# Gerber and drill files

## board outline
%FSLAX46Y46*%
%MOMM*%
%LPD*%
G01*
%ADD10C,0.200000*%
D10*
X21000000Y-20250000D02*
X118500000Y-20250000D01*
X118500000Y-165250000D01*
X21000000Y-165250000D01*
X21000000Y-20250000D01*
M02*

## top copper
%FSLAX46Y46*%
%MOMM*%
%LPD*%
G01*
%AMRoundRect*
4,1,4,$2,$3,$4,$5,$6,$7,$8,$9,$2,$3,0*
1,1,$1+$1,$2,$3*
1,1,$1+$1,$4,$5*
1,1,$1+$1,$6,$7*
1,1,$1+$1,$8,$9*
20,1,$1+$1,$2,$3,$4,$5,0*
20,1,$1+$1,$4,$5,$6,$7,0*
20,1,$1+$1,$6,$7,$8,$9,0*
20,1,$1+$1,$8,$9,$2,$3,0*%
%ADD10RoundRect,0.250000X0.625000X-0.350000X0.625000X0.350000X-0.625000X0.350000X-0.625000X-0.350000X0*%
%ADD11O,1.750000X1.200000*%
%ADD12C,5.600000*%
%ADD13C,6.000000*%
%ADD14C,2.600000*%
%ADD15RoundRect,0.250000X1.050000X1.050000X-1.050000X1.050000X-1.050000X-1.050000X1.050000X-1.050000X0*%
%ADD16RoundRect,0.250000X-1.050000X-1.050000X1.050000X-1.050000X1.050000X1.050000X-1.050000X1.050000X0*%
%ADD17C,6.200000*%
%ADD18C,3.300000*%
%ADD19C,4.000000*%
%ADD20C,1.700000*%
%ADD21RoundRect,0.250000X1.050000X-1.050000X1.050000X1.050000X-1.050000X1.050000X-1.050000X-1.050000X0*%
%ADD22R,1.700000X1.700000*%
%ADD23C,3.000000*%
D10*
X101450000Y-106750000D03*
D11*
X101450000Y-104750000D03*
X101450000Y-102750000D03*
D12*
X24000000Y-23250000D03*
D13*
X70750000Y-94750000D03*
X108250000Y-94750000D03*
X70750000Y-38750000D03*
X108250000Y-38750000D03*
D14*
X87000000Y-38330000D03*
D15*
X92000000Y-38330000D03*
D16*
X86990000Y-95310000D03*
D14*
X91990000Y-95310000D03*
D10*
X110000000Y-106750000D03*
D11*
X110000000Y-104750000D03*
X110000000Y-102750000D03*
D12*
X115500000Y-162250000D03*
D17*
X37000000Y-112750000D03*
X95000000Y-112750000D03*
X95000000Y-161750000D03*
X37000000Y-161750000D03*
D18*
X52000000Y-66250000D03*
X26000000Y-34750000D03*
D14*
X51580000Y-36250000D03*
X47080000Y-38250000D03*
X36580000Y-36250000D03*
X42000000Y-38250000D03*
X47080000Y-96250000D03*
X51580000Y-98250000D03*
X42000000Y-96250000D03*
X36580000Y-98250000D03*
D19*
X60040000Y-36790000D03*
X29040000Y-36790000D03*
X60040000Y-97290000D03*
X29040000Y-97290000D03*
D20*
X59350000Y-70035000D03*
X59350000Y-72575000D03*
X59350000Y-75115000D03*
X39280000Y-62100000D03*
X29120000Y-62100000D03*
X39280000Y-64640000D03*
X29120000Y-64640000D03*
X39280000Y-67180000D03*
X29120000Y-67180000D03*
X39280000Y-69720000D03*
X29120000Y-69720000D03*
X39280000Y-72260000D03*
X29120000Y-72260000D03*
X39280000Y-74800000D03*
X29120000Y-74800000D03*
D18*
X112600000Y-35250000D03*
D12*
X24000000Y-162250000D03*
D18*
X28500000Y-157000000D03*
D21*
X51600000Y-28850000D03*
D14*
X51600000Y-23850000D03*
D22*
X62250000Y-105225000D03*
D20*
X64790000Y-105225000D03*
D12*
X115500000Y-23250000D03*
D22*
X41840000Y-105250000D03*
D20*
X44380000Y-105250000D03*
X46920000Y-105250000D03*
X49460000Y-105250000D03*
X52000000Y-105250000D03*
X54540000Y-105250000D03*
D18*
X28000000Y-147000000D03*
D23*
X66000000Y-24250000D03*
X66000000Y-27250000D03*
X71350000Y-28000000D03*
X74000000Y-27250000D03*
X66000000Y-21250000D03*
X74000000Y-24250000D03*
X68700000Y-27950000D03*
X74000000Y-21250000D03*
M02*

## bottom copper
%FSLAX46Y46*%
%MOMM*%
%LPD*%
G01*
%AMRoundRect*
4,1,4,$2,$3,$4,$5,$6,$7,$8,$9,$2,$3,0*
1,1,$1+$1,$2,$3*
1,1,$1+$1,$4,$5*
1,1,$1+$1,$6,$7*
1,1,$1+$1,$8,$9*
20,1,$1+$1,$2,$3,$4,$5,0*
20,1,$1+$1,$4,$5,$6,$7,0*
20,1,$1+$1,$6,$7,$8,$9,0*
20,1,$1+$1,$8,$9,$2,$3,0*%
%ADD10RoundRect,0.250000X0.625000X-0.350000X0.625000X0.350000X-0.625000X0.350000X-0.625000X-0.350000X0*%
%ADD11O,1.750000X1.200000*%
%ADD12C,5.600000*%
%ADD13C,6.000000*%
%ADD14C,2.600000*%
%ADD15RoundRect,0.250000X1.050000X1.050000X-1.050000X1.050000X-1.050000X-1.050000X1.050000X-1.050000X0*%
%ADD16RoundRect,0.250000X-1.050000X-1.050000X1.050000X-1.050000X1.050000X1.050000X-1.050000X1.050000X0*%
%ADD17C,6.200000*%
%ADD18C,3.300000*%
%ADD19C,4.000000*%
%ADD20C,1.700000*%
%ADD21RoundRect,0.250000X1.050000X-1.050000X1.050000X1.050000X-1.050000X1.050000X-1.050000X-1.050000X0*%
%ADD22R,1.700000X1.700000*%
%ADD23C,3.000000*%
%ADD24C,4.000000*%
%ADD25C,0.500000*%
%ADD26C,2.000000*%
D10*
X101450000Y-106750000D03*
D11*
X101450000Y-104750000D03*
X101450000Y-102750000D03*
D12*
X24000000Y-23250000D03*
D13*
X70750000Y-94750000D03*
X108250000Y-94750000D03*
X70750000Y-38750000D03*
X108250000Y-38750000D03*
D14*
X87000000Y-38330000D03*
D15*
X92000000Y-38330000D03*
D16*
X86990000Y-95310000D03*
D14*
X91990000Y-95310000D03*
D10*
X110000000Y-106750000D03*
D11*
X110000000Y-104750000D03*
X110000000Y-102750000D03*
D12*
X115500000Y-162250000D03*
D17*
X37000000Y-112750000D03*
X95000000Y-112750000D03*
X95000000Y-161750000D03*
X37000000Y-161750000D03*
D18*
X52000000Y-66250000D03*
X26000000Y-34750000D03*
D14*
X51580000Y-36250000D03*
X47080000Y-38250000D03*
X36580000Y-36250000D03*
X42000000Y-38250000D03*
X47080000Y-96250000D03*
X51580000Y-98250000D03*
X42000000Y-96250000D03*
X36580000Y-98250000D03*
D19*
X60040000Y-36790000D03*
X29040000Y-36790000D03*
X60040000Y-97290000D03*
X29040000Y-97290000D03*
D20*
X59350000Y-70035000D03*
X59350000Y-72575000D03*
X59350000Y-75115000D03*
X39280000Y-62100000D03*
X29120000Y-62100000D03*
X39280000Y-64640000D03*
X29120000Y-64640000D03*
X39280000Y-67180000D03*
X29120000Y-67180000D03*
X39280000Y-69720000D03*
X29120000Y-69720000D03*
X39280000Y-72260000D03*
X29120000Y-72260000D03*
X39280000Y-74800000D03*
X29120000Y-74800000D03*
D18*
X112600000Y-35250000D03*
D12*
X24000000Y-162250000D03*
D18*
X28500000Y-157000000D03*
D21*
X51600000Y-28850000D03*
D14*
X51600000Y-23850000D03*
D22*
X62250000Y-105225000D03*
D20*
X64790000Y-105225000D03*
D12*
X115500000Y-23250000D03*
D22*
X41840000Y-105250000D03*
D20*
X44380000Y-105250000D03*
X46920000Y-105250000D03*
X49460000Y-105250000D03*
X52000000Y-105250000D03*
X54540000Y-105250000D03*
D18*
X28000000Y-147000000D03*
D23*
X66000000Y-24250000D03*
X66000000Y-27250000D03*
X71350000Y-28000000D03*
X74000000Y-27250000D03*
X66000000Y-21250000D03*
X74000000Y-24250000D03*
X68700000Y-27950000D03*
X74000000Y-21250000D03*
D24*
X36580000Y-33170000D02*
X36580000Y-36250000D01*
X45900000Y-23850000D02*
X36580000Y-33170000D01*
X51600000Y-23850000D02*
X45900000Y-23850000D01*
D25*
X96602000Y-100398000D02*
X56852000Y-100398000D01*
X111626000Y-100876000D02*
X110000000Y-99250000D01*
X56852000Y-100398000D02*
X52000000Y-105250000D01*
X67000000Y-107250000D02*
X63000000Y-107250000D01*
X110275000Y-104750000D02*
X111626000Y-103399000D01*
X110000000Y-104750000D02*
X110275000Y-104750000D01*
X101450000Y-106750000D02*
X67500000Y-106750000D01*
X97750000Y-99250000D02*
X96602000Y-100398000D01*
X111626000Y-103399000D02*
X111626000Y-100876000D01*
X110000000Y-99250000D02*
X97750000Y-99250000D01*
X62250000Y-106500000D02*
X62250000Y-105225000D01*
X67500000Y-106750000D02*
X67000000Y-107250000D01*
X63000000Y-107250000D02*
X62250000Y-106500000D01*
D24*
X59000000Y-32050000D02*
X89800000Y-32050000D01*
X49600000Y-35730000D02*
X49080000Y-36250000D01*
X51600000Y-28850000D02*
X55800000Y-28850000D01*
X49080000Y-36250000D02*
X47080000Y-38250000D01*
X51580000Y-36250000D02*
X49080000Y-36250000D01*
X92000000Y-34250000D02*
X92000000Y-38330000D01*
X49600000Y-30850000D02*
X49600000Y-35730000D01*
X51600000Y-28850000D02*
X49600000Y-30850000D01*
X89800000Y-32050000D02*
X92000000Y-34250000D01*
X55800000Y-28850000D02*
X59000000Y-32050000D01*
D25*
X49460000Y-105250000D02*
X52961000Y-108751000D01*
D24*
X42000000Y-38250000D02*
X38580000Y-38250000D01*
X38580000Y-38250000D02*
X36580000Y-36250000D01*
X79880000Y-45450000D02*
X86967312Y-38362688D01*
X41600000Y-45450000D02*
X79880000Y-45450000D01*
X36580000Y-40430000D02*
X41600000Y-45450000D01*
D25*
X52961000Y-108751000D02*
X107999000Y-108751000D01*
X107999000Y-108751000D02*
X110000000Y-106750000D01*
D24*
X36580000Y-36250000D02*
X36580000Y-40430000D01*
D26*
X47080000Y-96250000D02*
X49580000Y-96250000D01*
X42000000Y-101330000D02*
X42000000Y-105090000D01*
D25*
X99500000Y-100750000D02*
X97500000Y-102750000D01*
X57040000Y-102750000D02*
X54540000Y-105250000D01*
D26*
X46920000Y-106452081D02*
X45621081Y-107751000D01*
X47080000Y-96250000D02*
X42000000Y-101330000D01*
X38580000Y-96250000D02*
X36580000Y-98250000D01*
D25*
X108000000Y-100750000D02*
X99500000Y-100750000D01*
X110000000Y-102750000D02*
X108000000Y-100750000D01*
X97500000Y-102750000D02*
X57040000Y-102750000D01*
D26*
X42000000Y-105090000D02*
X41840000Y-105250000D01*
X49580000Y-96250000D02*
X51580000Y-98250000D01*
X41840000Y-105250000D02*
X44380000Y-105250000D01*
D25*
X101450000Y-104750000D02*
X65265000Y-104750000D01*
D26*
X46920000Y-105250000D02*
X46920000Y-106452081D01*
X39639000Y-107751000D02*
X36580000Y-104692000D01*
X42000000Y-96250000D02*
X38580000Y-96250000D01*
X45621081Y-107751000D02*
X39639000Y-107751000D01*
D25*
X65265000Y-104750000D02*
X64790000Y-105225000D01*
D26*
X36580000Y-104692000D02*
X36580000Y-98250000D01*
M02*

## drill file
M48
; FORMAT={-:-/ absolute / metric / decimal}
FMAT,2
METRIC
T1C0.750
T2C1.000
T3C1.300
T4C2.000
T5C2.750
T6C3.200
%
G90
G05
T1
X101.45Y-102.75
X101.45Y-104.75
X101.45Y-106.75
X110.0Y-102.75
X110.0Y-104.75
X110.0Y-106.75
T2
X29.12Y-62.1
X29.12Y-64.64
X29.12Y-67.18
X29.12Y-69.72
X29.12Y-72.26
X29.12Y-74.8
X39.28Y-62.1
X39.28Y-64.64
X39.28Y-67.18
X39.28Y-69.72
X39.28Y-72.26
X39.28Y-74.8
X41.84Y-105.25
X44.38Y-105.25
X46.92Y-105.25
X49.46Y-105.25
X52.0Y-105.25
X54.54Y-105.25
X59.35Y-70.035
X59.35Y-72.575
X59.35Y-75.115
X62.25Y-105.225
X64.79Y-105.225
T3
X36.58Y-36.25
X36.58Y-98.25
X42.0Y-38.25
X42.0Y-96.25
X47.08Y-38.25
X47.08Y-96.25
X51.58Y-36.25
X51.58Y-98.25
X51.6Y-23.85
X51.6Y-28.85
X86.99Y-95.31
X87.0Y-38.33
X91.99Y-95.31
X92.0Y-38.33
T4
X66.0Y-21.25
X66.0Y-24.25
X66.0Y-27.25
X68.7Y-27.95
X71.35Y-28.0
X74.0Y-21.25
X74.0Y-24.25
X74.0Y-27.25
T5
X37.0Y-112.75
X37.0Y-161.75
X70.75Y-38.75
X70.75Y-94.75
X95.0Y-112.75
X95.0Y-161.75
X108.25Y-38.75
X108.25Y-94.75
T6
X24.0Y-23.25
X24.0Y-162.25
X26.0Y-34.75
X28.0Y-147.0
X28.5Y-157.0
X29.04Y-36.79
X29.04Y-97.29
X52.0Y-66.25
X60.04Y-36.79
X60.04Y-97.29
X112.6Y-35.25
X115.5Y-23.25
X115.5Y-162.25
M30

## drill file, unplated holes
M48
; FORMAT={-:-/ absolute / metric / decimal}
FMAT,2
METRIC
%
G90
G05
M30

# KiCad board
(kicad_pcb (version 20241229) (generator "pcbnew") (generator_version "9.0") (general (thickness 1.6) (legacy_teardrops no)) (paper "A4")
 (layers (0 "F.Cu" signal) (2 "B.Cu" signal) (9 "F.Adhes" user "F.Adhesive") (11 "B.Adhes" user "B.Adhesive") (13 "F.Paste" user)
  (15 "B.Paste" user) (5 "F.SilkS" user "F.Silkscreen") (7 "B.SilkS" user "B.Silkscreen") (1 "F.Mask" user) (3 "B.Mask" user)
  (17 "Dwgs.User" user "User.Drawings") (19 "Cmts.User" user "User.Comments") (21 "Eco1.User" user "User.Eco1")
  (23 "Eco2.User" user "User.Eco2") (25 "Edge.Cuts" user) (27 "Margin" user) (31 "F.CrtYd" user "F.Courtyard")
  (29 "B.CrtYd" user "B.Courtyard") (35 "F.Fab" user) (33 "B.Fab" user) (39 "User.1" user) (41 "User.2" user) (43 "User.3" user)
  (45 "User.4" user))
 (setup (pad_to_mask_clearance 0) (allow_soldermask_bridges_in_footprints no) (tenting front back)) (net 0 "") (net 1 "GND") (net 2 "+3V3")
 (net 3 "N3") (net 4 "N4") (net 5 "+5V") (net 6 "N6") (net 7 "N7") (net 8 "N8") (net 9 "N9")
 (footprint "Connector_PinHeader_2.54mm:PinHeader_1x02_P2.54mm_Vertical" (layer "F.Cu") (at 62.25 105.225 90)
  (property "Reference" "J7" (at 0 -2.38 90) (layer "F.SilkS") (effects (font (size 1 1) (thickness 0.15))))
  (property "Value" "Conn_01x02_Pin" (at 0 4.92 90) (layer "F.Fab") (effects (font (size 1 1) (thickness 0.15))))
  (pad "1" thru_hole rect (at 0 0 90) (size 1.7 1.7) (drill 1) (layers "*.Cu" "*.Mask") (remove_unused_layers no) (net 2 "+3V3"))
  (pad "2" thru_hole circle (at 0 2.54 90) (size 1.7 1.7) (drill 1) (layers "*.Cu" "*.Mask") (remove_unused_layers no) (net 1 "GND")))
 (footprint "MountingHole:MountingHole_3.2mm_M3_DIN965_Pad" (layer "F.Cu") (at 24 23.25)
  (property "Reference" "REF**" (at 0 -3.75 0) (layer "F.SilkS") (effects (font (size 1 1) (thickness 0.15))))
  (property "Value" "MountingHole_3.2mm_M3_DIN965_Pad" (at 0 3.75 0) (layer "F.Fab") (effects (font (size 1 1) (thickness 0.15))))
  (pad "1" thru_hole circle (at 0 0) (size 5.6 5.6) (drill 3.2) (layers "*.Cu" "*.Mask") (remove_unused_layers no) (zone_connect 2)))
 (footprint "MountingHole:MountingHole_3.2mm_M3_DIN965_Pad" (layer "F.Cu") (at 24 162.25)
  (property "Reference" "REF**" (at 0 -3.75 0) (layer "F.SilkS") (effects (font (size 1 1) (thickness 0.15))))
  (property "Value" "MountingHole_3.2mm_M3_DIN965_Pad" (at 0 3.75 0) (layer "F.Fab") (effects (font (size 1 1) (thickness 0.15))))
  (pad "1" thru_hole circle (at 0 0) (size 5.6 5.6) (drill 3.2) (layers "*.Cu" "*.Mask") (remove_unused_layers no) (zone_connect 2)))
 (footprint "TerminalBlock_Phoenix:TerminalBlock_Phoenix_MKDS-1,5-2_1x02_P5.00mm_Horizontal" (layer "F.Cu") (at 51.6 28.85 90)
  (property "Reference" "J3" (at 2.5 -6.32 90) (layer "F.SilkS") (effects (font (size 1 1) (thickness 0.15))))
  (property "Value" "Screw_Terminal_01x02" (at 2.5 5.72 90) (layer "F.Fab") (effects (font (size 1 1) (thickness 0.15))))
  (pad "1" thru_hole roundrect (at 0 0 90) (size 2.6 2.6) (drill 1.3) (layers "*.Cu" "*.Mask") (remove_unused_layers no)
   (roundrect_rratio 0.096154) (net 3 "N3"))
  (pad "2" thru_hole circle (at 5 0 90) (size 2.6 2.6) (drill 1.3) (layers "*.Cu" "*.Mask") (remove_unused_layers no) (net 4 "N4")))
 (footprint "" (layer "F.Cu") (at 28 147)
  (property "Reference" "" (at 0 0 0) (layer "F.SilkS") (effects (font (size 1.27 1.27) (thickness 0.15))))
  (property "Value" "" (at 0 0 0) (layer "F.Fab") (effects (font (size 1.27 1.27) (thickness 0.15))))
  (pad "1" thru_hole circle (at 0 0) (size 3.3 3.3) (drill 3.2) (layers "*.Cu" "*.Mask") (remove_unused_layers no) (zone_connect 2)))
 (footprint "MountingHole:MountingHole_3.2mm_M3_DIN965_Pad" (layer "F.Cu") (at 112.6 35.25)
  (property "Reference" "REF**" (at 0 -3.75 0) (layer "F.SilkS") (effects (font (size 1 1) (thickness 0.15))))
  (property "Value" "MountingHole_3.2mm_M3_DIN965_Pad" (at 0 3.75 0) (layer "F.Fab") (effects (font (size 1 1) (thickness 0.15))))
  (pad "1" thru_hole circle (at 0 0) (size 3.3 3.3) (drill 3.2) (layers "*.Cu" "*.Mask") (remove_unused_layers no) (zone_connect 2)))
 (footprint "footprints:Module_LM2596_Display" (layer "F.Cu") (at 62.58 67.25 -90)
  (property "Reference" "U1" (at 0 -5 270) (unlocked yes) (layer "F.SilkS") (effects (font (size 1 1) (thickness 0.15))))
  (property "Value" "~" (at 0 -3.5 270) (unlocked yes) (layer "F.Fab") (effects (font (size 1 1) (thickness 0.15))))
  (pad "1" thru_hole circle (at -31 11 270) (size 2.6 2.6) (drill 1.3) (layers "*.Cu" "*.Mask") (remove_unused_layers no) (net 3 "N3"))
  (pad "1" thru_hole circle (at -29 15.5 270) (size 2.6 2.6) (drill 1.3) (layers "*.Cu" "*.Mask") (remove_unused_layers no) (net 3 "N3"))
  (pad "2" thru_hole circle (at -31 26 270) (size 2.6 2.6) (drill 1.3) (layers "*.Cu" "*.Mask") (remove_unused_layers no) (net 4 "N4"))
  (pad "2" thru_hole circle (at -29 20.58 270) (size 2.6 2.6) (drill 1.3) (layers "*.Cu" "*.Mask") (remove_unused_layers no) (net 4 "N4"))
  (pad "3" thru_hole circle (at 29 15.5 270) (size 2.6 2.6) (drill 1.3) (layers "*.Cu" "*.Mask") (remove_unused_layers no) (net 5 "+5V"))
  (pad "3" thru_hole circle (at 31 11 270) (size 2.6 2.6) (drill 1.3) (layers "*.Cu" "*.Mask") (remove_unused_layers no) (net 5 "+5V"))
  (pad "4" thru_hole circle (at 29 20.58 270) (size 2.6 2.6) (drill 1.3) (layers "*.Cu" "*.Mask") (remove_unused_layers no) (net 1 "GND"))
  (pad "4" thru_hole circle (at 31 26 270) (size 2.6 2.6) (drill 1.3) (layers "*.Cu" "*.Mask") (remove_unused_layers no) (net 1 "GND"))
  (pad "5" thru_hole circle (at -30.46 2.54 270) (size 4 4) (drill 3.2) (layers "*.Cu" "*.Mask") (remove_unused_layers no))
  (pad "5" thru_hole circle (at -30.46 33.54 270) (size 4 4) (drill 3.2) (layers "*.Cu" "*.Mask") (remove_unused_layers no))
  (pad "5" thru_hole circle (at 30.04 2.54 270) (size 4 4) (drill 3.2) (layers "*.Cu" "*.Mask") (remove_unused_layers no))
  (pad "5" thru_hole circle (at 30.04 33.54 270) (size 4 4) (drill 3.2) (layers "*.Cu" "*.Mask") (remove_unused_layers no))
  (pad "6" thru_hole circle (at 2.785 3.23 90) (size 1.7 1.7) (drill 1) (layers "*.Cu" "*.Mask") (remove_unused_layers no))
  (pad "7" thru_hole circle (at 5.325 3.23 90) (size 1.7 1.7) (drill 1) (layers "*.Cu" "*.Mask") (remove_unused_layers no))
  (pad "8" thru_hole circle (at 7.865 3.23 90) (size 1.7 1.7) (drill 1) (layers "*.Cu" "*.Mask") (remove_unused_layers no))
  (pad "9" thru_hole circle (at -5.15 23.3 270) (size 1.7 1.7) (drill 1) (layers "*.Cu" "*.Mask") (remove_unused_layers no))
  (pad "9" thru_hole circle (at -5.15 33.46 270) (size 1.7 1.7) (drill 1) (layers "*.Cu" "*.Mask") (remove_unused_layers no))
  (pad "9" thru_hole circle (at -2.61 23.3 270) (size 1.7 1.7) (drill 1) (layers "*.Cu" "*.Mask") (remove_unused_layers no))
  (pad "9" thru_hole circle (at -2.61 33.46 270) (size 1.7 1.7) (drill 1) (layers "*.Cu" "*.Mask") (remove_unused_layers no))
  (pad "9" thru_hole circle (at -0.07 23.3 270) (size 1.7 1.7) (drill 1) (layers "*.Cu" "*.Mask") (remove_unused_layers no))
  (pad "9" thru_hole circle (at -0.07 33.46 270) (size 1.7 1.7) (drill 1) (layers "*.Cu" "*.Mask") (remove_unused_layers no))
  (pad "9" thru_hole circle (at 2.47 23.3 270) (size 1.7 1.7) (drill 1) (layers "*.Cu" "*.Mask" "Eco1.User") (remove_unused_layers no))
  (pad "9" thru_hole circle (at 2.47 33.46 270) (size 1.7 1.7) (drill 1) (layers "*.Cu" "*.Mask") (remove_unused_layers no))
  (pad "9" thru_hole circle (at 5.01 23.3 270) (size 1.7 1.7) (drill 1) (layers "*.Cu" "*.Mask") (remove_unused_layers no))
  (pad "9" thru_hole circle (at 5.01 33.46 270) (size 1.7 1.7) (drill 1) (layers "*.Cu" "*.Mask") (remove_unused_layers no))
  (pad "9" thru_hole circle (at 7.55 23.3 270) (size 1.7 1.7) (drill 1) (layers "*.Cu" "*.Mask") (remove_unused_layers no))
  (pad "9" thru_hole circle (at 7.55 33.46 270) (size 1.7 1.7) (drill 1) (layers "*.Cu" "*.Mask") (remove_unused_layers no)))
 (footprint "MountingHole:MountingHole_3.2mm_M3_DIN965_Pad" (layer "F.Cu") (at 115.5 162.25)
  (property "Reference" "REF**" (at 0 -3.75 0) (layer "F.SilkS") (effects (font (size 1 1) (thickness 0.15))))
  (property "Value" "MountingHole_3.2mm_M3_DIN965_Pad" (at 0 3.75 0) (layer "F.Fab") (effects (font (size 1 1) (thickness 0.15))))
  (pad "1" thru_hole circle (at 0 0) (size 5.6 5.6) (drill 3.2) (layers "*.Cu" "*.Mask") (remove_unused_layers no) (zone_connect 2)))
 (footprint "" (layer "F.Cu") (at 28.5 157)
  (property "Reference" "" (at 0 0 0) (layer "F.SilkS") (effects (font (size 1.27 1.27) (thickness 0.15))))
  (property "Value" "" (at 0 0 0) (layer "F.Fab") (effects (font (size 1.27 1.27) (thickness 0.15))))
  (pad "1" thru_hole circle (at 0 0) (size 3.3 3.3) (drill 3.2) (layers "*.Cu" "*.Mask") (remove_unused_layers no) (zone_connect 2)))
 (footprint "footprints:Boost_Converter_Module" (layer "F.Cu") (at 89.5 66.75 90)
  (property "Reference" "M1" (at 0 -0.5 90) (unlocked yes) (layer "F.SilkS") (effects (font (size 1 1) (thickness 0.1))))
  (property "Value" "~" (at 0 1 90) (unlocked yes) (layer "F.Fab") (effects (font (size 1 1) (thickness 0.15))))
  (pad "" thru_hole circle (at -28 -18.75 90) (size 6 6) (drill 2.75) (layers "*.Cu" "*.Mask") (remove_unused_layers no))
  (pad "" thru_hole circle (at -28 18.75 90) (size 6 6) (drill 2.75) (layers "*.Cu" "*.Mask") (remove_unused_layers no))
  (pad "" thru_hole circle (at 28 -18.75 90) (size 6 6) (drill 2.75) (layers "*.Cu" "*.Mask") (remove_unused_layers no))
  (pad "" thru_hole circle (at 28 18.75 90) (size 6 6) (drill 2.75) (layers "*.Cu" "*.Mask") (remove_unused_layers no))
  (pad "1" thru_hole circle (at 28.42 -2.5 180) (size 2.6 2.6) (drill 1.3) (layers "*.Cu" "*.Mask") (remove_unused_layers no) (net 4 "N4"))
  (pad "2" thru_hole roundrect (at 28.42 2.5 180) (size 2.6 2.6) (drill 1.3) (layers "*.Cu" "*.Mask") (remove_unused_layers no)
   (roundrect_rratio 0.096154) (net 3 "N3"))
  (pad "3" thru_hole roundrect (at -28.56 -2.51) (size 2.6 2.6) (drill 1.3) (layers "*.Cu" "*.Mask") (remove_unused_layers no)
   (roundrect_rratio 0.096154))
  (pad "4" thru_hole circle (at -28.56 2.49) (size 2.6 2.6) (drill 1.3) (layers "*.Cu" "*.Mask") (remove_unused_layers no)))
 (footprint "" (layer "F.Cu") (at 26 34.75)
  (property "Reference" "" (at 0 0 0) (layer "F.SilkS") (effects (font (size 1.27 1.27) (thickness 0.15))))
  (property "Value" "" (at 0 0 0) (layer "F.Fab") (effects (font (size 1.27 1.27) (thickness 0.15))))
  (pad "1" thru_hole circle (at 0 0) (size 3.3 3.3) (drill 3.2) (layers "*.Cu" "*.Mask") (remove_unused_layers no) (zone_connect 2)))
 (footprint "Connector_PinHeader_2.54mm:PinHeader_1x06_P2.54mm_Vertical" (layer "F.Cu") (at 41.84 105.25 90)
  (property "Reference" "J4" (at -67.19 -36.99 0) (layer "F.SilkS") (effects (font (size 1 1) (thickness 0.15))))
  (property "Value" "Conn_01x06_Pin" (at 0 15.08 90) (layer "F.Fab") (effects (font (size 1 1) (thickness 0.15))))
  (pad "1" thru_hole rect (at 0 0 90) (size 1.7 1.7) (drill 1) (layers "*.Cu" "*.Mask") (remove_unused_layers no) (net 5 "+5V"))
  (pad "2" thru_hole circle (at 0 2.54 90) (size 1.7 1.7) (drill 1) (layers "*.Cu" "*.Mask") (remove_unused_layers no) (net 5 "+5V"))
  (pad "3" thru_hole circle (at 0 5.08 90) (size 1.7 1.7) (drill 1) (layers "*.Cu" "*.Mask") (remove_unused_layers no) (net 1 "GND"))
  (pad "4" thru_hole circle (at 0 7.62 90) (size 1.7 1.7) (drill 1) (layers "*.Cu" "*.Mask") (remove_unused_layers no) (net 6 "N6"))
  (pad "5" thru_hole circle (at 0 10.16 90) (size 1.7 1.7) (drill 1) (layers "*.Cu" "*.Mask") (remove_unused_layers no) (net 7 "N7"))
  (pad "6" thru_hole circle (at 0 12.7 90) (size 1.7 1.7) (drill 1) (layers "*.Cu" "*.Mask") (remove_unused_layers no) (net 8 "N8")))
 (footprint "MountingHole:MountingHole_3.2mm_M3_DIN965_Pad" (layer "F.Cu") (at 115.5 23.25)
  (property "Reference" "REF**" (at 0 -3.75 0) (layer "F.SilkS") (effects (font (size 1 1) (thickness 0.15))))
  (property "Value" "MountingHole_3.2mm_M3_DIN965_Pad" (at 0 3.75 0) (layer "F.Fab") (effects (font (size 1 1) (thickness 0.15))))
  (pad "1" thru_hole circle (at 0 0) (size 5.6 5.6) (drill 3.2) (layers "*.Cu" "*.Mask") (remove_unused_layers no) (zone_connect 2)))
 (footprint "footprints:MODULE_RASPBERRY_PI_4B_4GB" (layer "F.Cu") (at 76 137.25)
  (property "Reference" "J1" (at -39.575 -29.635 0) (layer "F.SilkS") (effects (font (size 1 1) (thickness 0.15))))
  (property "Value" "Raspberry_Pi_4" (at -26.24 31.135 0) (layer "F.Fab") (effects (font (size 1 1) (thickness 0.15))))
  (pad "S1" thru_hole circle (at -39 -24.5) (size 6.2 6.2) (drill 2.75) (layers "*.Cu" "*.Mask") (remove_unused_layers no)
   (solder_mask_margin 0.102))
  (pad "S2" thru_hole circle (at 19 -24.5) (size 6.2 6.2) (drill 2.75) (layers "*.Cu" "*.Mask") (remove_unused_layers no)
   (solder_mask_margin 0.102))
  (pad "S3" thru_hole circle (at 19 24.5) (size 6.2 6.2) (drill 2.75) (layers "*.Cu" "*.Mask") (remove_unused_layers no)
   (solder_mask_margin 0.102))
  (pad "S4" thru_hole circle (at -39 24.5) (size 6.2 6.2) (drill 2.75) (layers "*.Cu" "*.Mask") (remove_unused_layers no)
   (solder_mask_margin 0.102)))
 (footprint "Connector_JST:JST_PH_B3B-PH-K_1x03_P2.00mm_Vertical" (layer "F.Cu") (at 101.45 106.75 90)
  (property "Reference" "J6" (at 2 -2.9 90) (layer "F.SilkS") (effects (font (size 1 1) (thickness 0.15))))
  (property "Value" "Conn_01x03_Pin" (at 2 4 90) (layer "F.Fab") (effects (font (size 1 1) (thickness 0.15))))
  (pad "1" thru_hole roundrect (at 0 0 90) (size 1.2 1.75) (drill 0.75) (layers "*.Cu" "*.Mask") (remove_unused_layers no)
   (roundrect_rratio 0.208333) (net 2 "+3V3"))
  (pad "2" thru_hole oval (at 2 0 90) (size 1.2 1.75) (drill 0.75) (layers "*.Cu" "*.Mask") (remove_unused_layers no) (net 1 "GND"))
  (pad "3" thru_hole oval (at 4 0 90) (size 1.2 1.75) (drill 0.75) (layers "*.Cu" "*.Mask") (remove_unused_layers no) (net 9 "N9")))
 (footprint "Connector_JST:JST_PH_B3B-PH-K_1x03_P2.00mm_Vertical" (layer "F.Cu") (at 110 106.75 90)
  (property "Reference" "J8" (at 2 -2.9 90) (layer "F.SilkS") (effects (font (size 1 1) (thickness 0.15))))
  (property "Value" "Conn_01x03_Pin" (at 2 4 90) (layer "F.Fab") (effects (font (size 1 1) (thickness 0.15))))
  (pad "1" thru_hole roundrect (at 0 0 90) (size 1.2 1.75) (drill 0.75) (layers "*.Cu" "*.Mask") (remove_unused_layers no)
   (roundrect_rratio 0.208333) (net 6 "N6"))
  (pad "2" thru_hole oval (at 2 0 90) (size 1.2 1.75) (drill 0.75) (layers "*.Cu" "*.Mask") (remove_unused_layers no) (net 7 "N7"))
  (pad "3" thru_hole oval (at 4 0 90) (size 1.2 1.75) (drill 0.75) (layers "*.Cu" "*.Mask") (remove_unused_layers no) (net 8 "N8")))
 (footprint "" (layer "F.Cu") (at 52 66.25)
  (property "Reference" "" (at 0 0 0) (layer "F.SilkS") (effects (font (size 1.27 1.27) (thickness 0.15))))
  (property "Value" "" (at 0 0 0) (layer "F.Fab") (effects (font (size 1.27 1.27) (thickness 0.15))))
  (pad "1" thru_hole circle (at 0 0) (size 3.3 3.3) (drill 3.2) (layers "*.Cu" "*.Mask") (remove_unused_layers no) (zone_connect 2)))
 (gr_rect (start 21 20.25) (end 118.5 165.25) (stroke (width 0.2) (type solid)) (fill no) (layer "Edge.Cuts"))
 (via (at 66 27.25) (size 3) (drill 2) (layers "F.Cu" "B.Cu") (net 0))
 (via (at 74 27.25) (size 3) (drill 2) (layers "F.Cu" "B.Cu") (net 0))
 (via (at 74 21.25) (size 3) (drill 2) (layers "F.Cu" "B.Cu") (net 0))
 (via (at 66 24.25) (size 3) (drill 2) (layers "F.Cu" "B.Cu") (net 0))
 (via (at 71.35 28) (size 3) (drill 2) (layers "F.Cu" "B.Cu") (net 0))
 (via (at 66 21.25) (size 3) (drill 2) (layers "F.Cu" "B.Cu") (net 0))
 (via (at 74 24.25) (size 3) (drill 2) (layers "F.Cu" "B.Cu") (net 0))
 (via (at 68.7 27.95) (size 3) (drill 2) (layers "F.Cu" "B.Cu") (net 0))
 (segment (start 101.45 104.75) (end 65.265 104.75) (width 0.5) (layer "B.Cu") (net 1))
 (segment (start 46.92 105.25) (end 46.92 106.452081) (width 2) (layer "B.Cu") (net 1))
 (segment (start 46.92 106.452081) (end 45.621081 107.751) (width 2) (layer "B.Cu") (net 1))
 (segment (start 65.265 104.75) (end 64.79 105.225) (width 0.5) (layer "B.Cu") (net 1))
 (segment (start 39.639 107.751) (end 36.58 104.692) (width 2) (layer "B.Cu") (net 1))
 (segment (start 38.58 96.25) (end 36.58 98.25) (width 2) (layer "B.Cu") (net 1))
 (segment (start 36.58 104.692) (end 36.58 98.25) (width 2) (layer "B.Cu") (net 1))
 (segment (start 42 96.25) (end 38.58 96.25) (width 2) (layer "B.Cu") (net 1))
 (segment (start 45.621081 107.751) (end 39.639 107.751) (width 2) (layer "B.Cu") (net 1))
 (segment (start 42 105.09) (end 41.84 105.25) (width 2) (layer "B.Cu") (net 5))
 (segment (start 49.58 96.25) (end 51.58 98.25) (width 2) (layer "B.Cu") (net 5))
 (segment (start 47.08 96.25) (end 42 101.33) (width 2) (layer "B.Cu") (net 5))
 (segment (start 41.84 105.25) (end 44.38 105.25) (width 2) (layer "B.Cu") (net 5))
 (segment (start 42 101.33) (end 42 105.09) (width 2) (layer "B.Cu") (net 5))
 (segment (start 47.08 96.25) (end 49.58 96.25) (width 2) (layer "B.Cu") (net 5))
 (segment (start 99.5 100.75) (end 97.5 102.75) (width 0.5) (layer "B.Cu") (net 8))
 (segment (start 108 100.75) (end 99.5 100.75) (width 0.5) (layer "B.Cu") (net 8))
 (segment (start 57.04 102.75) (end 54.54 105.25) (width 0.5) (layer "B.Cu") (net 8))
 (segment (start 97.5 102.75) (end 57.04 102.75) (width 0.5) (layer "B.Cu") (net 8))
 (segment (start 110 102.75) (end 108 100.75) (width 0.5) (layer "B.Cu") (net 8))
 (segment (start 36.58 36.25) (end 36.58 40.43) (width 4) (layer "B.Cu") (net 4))
 (segment (start 79.88 45.45) (end 86.967312 38.362688) (width 4) (layer "B.Cu") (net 4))
 (segment (start 51.6 23.85) (end 45.9 23.85) (width 4) (layer "B.Cu") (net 4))
 (segment (start 36.58 33.17) (end 36.58 36.25) (width 4) (layer "B.Cu") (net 4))
 (segment (start 41.6 45.45) (end 79.88 45.45) (width 4) (layer "B.Cu") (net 4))
 (segment (start 38.58 38.25) (end 36.58 36.25) (width 4) (layer "B.Cu") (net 4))
 (segment (start 42 38.25) (end 38.58 38.25) (width 4) (layer "B.Cu") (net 4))
 (segment (start 36.58 40.43) (end 41.6 45.45) (width 4) (layer "B.Cu") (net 4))
 (segment (start 45.9 23.85) (end 36.58 33.17) (width 4) (layer "B.Cu") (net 4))
 (segment (start 49.46 105.25) (end 52.961 108.751) (width 0.5) (layer "B.Cu") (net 6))
 (segment (start 52.961 108.751) (end 107.999 108.751) (width 0.5) (layer "B.Cu") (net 6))
 (segment (start 107.999 108.751) (end 110 106.75) (width 0.5) (layer "B.Cu") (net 6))
 (segment (start 89.8 32.05) (end 92 34.25) (width 4) (layer "B.Cu") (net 3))
 (segment (start 92 34.25) (end 92 38.33) (width 4) (layer "B.Cu") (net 3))
 (segment (start 51.6 28.85) (end 49.6 30.85) (width 4) (layer "B.Cu") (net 3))
 (segment (start 55.8 28.85) (end 59 32.05) (width 4) (layer "B.Cu") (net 3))
 (segment (start 49.6 35.73) (end 49.08 36.25) (width 4) (layer "B.Cu") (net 3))
 (segment (start 49.08 36.25) (end 47.08 38.25) (width 4) (layer "B.Cu") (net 3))
 (segment (start 59 32.05) (end 89.8 32.05) (width 4) (layer "B.Cu") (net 3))
 (segment (start 49.6 30.85) (end 49.6 35.73) (width 4) (layer "B.Cu") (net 3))
 (segment (start 51.58 36.25) (end 49.08 36.25) (width 4) (layer "B.Cu") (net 3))
 (segment (start 51.6 28.85) (end 55.8 28.85) (width 4) (layer "B.Cu") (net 3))
 (segment (start 67.5 106.75) (end 67 107.25) (width 0.5) (layer "B.Cu") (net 2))
 (segment (start 63 107.25) (end 62.25 106.5) (width 0.5) (layer "B.Cu") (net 2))
 (segment (start 67 107.25) (end 63 107.25) (width 0.5) (layer "B.Cu") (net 2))
 (segment (start 62.25 106.5) (end 62.25 105.225) (width 0.5) (layer "B.Cu") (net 2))
 (segment (start 101.45 106.75) (end 67.5 106.75) (width 0.5) (layer "B.Cu") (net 2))
 (segment (start 110.275 104.75) (end 111.626 103.399) (width 0.5) (layer "B.Cu") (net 7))
 (segment (start 97.75 99.25) (end 96.602 100.398) (width 0.5) (layer "B.Cu") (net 7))
 (segment (start 56.852 100.398) (end 52 105.25) (width 0.5) (layer "B.Cu") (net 7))
 (segment (start 111.626 100.876) (end 110 99.25) (width 0.5) (layer "B.Cu") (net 7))
 (segment (start 110 99.25) (end 97.75 99.25) (width 0.5) (layer "B.Cu") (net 7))
 (segment (start 96.602 100.398) (end 56.852 100.398) (width 0.5) (layer "B.Cu") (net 7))
 (segment (start 111.626 103.399) (end 111.626 100.876) (width 0.5) (layer "B.Cu") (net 7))
 (segment (start 110 104.75) (end 110.275 104.75) (width 0.5) (layer "B.Cu") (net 7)))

